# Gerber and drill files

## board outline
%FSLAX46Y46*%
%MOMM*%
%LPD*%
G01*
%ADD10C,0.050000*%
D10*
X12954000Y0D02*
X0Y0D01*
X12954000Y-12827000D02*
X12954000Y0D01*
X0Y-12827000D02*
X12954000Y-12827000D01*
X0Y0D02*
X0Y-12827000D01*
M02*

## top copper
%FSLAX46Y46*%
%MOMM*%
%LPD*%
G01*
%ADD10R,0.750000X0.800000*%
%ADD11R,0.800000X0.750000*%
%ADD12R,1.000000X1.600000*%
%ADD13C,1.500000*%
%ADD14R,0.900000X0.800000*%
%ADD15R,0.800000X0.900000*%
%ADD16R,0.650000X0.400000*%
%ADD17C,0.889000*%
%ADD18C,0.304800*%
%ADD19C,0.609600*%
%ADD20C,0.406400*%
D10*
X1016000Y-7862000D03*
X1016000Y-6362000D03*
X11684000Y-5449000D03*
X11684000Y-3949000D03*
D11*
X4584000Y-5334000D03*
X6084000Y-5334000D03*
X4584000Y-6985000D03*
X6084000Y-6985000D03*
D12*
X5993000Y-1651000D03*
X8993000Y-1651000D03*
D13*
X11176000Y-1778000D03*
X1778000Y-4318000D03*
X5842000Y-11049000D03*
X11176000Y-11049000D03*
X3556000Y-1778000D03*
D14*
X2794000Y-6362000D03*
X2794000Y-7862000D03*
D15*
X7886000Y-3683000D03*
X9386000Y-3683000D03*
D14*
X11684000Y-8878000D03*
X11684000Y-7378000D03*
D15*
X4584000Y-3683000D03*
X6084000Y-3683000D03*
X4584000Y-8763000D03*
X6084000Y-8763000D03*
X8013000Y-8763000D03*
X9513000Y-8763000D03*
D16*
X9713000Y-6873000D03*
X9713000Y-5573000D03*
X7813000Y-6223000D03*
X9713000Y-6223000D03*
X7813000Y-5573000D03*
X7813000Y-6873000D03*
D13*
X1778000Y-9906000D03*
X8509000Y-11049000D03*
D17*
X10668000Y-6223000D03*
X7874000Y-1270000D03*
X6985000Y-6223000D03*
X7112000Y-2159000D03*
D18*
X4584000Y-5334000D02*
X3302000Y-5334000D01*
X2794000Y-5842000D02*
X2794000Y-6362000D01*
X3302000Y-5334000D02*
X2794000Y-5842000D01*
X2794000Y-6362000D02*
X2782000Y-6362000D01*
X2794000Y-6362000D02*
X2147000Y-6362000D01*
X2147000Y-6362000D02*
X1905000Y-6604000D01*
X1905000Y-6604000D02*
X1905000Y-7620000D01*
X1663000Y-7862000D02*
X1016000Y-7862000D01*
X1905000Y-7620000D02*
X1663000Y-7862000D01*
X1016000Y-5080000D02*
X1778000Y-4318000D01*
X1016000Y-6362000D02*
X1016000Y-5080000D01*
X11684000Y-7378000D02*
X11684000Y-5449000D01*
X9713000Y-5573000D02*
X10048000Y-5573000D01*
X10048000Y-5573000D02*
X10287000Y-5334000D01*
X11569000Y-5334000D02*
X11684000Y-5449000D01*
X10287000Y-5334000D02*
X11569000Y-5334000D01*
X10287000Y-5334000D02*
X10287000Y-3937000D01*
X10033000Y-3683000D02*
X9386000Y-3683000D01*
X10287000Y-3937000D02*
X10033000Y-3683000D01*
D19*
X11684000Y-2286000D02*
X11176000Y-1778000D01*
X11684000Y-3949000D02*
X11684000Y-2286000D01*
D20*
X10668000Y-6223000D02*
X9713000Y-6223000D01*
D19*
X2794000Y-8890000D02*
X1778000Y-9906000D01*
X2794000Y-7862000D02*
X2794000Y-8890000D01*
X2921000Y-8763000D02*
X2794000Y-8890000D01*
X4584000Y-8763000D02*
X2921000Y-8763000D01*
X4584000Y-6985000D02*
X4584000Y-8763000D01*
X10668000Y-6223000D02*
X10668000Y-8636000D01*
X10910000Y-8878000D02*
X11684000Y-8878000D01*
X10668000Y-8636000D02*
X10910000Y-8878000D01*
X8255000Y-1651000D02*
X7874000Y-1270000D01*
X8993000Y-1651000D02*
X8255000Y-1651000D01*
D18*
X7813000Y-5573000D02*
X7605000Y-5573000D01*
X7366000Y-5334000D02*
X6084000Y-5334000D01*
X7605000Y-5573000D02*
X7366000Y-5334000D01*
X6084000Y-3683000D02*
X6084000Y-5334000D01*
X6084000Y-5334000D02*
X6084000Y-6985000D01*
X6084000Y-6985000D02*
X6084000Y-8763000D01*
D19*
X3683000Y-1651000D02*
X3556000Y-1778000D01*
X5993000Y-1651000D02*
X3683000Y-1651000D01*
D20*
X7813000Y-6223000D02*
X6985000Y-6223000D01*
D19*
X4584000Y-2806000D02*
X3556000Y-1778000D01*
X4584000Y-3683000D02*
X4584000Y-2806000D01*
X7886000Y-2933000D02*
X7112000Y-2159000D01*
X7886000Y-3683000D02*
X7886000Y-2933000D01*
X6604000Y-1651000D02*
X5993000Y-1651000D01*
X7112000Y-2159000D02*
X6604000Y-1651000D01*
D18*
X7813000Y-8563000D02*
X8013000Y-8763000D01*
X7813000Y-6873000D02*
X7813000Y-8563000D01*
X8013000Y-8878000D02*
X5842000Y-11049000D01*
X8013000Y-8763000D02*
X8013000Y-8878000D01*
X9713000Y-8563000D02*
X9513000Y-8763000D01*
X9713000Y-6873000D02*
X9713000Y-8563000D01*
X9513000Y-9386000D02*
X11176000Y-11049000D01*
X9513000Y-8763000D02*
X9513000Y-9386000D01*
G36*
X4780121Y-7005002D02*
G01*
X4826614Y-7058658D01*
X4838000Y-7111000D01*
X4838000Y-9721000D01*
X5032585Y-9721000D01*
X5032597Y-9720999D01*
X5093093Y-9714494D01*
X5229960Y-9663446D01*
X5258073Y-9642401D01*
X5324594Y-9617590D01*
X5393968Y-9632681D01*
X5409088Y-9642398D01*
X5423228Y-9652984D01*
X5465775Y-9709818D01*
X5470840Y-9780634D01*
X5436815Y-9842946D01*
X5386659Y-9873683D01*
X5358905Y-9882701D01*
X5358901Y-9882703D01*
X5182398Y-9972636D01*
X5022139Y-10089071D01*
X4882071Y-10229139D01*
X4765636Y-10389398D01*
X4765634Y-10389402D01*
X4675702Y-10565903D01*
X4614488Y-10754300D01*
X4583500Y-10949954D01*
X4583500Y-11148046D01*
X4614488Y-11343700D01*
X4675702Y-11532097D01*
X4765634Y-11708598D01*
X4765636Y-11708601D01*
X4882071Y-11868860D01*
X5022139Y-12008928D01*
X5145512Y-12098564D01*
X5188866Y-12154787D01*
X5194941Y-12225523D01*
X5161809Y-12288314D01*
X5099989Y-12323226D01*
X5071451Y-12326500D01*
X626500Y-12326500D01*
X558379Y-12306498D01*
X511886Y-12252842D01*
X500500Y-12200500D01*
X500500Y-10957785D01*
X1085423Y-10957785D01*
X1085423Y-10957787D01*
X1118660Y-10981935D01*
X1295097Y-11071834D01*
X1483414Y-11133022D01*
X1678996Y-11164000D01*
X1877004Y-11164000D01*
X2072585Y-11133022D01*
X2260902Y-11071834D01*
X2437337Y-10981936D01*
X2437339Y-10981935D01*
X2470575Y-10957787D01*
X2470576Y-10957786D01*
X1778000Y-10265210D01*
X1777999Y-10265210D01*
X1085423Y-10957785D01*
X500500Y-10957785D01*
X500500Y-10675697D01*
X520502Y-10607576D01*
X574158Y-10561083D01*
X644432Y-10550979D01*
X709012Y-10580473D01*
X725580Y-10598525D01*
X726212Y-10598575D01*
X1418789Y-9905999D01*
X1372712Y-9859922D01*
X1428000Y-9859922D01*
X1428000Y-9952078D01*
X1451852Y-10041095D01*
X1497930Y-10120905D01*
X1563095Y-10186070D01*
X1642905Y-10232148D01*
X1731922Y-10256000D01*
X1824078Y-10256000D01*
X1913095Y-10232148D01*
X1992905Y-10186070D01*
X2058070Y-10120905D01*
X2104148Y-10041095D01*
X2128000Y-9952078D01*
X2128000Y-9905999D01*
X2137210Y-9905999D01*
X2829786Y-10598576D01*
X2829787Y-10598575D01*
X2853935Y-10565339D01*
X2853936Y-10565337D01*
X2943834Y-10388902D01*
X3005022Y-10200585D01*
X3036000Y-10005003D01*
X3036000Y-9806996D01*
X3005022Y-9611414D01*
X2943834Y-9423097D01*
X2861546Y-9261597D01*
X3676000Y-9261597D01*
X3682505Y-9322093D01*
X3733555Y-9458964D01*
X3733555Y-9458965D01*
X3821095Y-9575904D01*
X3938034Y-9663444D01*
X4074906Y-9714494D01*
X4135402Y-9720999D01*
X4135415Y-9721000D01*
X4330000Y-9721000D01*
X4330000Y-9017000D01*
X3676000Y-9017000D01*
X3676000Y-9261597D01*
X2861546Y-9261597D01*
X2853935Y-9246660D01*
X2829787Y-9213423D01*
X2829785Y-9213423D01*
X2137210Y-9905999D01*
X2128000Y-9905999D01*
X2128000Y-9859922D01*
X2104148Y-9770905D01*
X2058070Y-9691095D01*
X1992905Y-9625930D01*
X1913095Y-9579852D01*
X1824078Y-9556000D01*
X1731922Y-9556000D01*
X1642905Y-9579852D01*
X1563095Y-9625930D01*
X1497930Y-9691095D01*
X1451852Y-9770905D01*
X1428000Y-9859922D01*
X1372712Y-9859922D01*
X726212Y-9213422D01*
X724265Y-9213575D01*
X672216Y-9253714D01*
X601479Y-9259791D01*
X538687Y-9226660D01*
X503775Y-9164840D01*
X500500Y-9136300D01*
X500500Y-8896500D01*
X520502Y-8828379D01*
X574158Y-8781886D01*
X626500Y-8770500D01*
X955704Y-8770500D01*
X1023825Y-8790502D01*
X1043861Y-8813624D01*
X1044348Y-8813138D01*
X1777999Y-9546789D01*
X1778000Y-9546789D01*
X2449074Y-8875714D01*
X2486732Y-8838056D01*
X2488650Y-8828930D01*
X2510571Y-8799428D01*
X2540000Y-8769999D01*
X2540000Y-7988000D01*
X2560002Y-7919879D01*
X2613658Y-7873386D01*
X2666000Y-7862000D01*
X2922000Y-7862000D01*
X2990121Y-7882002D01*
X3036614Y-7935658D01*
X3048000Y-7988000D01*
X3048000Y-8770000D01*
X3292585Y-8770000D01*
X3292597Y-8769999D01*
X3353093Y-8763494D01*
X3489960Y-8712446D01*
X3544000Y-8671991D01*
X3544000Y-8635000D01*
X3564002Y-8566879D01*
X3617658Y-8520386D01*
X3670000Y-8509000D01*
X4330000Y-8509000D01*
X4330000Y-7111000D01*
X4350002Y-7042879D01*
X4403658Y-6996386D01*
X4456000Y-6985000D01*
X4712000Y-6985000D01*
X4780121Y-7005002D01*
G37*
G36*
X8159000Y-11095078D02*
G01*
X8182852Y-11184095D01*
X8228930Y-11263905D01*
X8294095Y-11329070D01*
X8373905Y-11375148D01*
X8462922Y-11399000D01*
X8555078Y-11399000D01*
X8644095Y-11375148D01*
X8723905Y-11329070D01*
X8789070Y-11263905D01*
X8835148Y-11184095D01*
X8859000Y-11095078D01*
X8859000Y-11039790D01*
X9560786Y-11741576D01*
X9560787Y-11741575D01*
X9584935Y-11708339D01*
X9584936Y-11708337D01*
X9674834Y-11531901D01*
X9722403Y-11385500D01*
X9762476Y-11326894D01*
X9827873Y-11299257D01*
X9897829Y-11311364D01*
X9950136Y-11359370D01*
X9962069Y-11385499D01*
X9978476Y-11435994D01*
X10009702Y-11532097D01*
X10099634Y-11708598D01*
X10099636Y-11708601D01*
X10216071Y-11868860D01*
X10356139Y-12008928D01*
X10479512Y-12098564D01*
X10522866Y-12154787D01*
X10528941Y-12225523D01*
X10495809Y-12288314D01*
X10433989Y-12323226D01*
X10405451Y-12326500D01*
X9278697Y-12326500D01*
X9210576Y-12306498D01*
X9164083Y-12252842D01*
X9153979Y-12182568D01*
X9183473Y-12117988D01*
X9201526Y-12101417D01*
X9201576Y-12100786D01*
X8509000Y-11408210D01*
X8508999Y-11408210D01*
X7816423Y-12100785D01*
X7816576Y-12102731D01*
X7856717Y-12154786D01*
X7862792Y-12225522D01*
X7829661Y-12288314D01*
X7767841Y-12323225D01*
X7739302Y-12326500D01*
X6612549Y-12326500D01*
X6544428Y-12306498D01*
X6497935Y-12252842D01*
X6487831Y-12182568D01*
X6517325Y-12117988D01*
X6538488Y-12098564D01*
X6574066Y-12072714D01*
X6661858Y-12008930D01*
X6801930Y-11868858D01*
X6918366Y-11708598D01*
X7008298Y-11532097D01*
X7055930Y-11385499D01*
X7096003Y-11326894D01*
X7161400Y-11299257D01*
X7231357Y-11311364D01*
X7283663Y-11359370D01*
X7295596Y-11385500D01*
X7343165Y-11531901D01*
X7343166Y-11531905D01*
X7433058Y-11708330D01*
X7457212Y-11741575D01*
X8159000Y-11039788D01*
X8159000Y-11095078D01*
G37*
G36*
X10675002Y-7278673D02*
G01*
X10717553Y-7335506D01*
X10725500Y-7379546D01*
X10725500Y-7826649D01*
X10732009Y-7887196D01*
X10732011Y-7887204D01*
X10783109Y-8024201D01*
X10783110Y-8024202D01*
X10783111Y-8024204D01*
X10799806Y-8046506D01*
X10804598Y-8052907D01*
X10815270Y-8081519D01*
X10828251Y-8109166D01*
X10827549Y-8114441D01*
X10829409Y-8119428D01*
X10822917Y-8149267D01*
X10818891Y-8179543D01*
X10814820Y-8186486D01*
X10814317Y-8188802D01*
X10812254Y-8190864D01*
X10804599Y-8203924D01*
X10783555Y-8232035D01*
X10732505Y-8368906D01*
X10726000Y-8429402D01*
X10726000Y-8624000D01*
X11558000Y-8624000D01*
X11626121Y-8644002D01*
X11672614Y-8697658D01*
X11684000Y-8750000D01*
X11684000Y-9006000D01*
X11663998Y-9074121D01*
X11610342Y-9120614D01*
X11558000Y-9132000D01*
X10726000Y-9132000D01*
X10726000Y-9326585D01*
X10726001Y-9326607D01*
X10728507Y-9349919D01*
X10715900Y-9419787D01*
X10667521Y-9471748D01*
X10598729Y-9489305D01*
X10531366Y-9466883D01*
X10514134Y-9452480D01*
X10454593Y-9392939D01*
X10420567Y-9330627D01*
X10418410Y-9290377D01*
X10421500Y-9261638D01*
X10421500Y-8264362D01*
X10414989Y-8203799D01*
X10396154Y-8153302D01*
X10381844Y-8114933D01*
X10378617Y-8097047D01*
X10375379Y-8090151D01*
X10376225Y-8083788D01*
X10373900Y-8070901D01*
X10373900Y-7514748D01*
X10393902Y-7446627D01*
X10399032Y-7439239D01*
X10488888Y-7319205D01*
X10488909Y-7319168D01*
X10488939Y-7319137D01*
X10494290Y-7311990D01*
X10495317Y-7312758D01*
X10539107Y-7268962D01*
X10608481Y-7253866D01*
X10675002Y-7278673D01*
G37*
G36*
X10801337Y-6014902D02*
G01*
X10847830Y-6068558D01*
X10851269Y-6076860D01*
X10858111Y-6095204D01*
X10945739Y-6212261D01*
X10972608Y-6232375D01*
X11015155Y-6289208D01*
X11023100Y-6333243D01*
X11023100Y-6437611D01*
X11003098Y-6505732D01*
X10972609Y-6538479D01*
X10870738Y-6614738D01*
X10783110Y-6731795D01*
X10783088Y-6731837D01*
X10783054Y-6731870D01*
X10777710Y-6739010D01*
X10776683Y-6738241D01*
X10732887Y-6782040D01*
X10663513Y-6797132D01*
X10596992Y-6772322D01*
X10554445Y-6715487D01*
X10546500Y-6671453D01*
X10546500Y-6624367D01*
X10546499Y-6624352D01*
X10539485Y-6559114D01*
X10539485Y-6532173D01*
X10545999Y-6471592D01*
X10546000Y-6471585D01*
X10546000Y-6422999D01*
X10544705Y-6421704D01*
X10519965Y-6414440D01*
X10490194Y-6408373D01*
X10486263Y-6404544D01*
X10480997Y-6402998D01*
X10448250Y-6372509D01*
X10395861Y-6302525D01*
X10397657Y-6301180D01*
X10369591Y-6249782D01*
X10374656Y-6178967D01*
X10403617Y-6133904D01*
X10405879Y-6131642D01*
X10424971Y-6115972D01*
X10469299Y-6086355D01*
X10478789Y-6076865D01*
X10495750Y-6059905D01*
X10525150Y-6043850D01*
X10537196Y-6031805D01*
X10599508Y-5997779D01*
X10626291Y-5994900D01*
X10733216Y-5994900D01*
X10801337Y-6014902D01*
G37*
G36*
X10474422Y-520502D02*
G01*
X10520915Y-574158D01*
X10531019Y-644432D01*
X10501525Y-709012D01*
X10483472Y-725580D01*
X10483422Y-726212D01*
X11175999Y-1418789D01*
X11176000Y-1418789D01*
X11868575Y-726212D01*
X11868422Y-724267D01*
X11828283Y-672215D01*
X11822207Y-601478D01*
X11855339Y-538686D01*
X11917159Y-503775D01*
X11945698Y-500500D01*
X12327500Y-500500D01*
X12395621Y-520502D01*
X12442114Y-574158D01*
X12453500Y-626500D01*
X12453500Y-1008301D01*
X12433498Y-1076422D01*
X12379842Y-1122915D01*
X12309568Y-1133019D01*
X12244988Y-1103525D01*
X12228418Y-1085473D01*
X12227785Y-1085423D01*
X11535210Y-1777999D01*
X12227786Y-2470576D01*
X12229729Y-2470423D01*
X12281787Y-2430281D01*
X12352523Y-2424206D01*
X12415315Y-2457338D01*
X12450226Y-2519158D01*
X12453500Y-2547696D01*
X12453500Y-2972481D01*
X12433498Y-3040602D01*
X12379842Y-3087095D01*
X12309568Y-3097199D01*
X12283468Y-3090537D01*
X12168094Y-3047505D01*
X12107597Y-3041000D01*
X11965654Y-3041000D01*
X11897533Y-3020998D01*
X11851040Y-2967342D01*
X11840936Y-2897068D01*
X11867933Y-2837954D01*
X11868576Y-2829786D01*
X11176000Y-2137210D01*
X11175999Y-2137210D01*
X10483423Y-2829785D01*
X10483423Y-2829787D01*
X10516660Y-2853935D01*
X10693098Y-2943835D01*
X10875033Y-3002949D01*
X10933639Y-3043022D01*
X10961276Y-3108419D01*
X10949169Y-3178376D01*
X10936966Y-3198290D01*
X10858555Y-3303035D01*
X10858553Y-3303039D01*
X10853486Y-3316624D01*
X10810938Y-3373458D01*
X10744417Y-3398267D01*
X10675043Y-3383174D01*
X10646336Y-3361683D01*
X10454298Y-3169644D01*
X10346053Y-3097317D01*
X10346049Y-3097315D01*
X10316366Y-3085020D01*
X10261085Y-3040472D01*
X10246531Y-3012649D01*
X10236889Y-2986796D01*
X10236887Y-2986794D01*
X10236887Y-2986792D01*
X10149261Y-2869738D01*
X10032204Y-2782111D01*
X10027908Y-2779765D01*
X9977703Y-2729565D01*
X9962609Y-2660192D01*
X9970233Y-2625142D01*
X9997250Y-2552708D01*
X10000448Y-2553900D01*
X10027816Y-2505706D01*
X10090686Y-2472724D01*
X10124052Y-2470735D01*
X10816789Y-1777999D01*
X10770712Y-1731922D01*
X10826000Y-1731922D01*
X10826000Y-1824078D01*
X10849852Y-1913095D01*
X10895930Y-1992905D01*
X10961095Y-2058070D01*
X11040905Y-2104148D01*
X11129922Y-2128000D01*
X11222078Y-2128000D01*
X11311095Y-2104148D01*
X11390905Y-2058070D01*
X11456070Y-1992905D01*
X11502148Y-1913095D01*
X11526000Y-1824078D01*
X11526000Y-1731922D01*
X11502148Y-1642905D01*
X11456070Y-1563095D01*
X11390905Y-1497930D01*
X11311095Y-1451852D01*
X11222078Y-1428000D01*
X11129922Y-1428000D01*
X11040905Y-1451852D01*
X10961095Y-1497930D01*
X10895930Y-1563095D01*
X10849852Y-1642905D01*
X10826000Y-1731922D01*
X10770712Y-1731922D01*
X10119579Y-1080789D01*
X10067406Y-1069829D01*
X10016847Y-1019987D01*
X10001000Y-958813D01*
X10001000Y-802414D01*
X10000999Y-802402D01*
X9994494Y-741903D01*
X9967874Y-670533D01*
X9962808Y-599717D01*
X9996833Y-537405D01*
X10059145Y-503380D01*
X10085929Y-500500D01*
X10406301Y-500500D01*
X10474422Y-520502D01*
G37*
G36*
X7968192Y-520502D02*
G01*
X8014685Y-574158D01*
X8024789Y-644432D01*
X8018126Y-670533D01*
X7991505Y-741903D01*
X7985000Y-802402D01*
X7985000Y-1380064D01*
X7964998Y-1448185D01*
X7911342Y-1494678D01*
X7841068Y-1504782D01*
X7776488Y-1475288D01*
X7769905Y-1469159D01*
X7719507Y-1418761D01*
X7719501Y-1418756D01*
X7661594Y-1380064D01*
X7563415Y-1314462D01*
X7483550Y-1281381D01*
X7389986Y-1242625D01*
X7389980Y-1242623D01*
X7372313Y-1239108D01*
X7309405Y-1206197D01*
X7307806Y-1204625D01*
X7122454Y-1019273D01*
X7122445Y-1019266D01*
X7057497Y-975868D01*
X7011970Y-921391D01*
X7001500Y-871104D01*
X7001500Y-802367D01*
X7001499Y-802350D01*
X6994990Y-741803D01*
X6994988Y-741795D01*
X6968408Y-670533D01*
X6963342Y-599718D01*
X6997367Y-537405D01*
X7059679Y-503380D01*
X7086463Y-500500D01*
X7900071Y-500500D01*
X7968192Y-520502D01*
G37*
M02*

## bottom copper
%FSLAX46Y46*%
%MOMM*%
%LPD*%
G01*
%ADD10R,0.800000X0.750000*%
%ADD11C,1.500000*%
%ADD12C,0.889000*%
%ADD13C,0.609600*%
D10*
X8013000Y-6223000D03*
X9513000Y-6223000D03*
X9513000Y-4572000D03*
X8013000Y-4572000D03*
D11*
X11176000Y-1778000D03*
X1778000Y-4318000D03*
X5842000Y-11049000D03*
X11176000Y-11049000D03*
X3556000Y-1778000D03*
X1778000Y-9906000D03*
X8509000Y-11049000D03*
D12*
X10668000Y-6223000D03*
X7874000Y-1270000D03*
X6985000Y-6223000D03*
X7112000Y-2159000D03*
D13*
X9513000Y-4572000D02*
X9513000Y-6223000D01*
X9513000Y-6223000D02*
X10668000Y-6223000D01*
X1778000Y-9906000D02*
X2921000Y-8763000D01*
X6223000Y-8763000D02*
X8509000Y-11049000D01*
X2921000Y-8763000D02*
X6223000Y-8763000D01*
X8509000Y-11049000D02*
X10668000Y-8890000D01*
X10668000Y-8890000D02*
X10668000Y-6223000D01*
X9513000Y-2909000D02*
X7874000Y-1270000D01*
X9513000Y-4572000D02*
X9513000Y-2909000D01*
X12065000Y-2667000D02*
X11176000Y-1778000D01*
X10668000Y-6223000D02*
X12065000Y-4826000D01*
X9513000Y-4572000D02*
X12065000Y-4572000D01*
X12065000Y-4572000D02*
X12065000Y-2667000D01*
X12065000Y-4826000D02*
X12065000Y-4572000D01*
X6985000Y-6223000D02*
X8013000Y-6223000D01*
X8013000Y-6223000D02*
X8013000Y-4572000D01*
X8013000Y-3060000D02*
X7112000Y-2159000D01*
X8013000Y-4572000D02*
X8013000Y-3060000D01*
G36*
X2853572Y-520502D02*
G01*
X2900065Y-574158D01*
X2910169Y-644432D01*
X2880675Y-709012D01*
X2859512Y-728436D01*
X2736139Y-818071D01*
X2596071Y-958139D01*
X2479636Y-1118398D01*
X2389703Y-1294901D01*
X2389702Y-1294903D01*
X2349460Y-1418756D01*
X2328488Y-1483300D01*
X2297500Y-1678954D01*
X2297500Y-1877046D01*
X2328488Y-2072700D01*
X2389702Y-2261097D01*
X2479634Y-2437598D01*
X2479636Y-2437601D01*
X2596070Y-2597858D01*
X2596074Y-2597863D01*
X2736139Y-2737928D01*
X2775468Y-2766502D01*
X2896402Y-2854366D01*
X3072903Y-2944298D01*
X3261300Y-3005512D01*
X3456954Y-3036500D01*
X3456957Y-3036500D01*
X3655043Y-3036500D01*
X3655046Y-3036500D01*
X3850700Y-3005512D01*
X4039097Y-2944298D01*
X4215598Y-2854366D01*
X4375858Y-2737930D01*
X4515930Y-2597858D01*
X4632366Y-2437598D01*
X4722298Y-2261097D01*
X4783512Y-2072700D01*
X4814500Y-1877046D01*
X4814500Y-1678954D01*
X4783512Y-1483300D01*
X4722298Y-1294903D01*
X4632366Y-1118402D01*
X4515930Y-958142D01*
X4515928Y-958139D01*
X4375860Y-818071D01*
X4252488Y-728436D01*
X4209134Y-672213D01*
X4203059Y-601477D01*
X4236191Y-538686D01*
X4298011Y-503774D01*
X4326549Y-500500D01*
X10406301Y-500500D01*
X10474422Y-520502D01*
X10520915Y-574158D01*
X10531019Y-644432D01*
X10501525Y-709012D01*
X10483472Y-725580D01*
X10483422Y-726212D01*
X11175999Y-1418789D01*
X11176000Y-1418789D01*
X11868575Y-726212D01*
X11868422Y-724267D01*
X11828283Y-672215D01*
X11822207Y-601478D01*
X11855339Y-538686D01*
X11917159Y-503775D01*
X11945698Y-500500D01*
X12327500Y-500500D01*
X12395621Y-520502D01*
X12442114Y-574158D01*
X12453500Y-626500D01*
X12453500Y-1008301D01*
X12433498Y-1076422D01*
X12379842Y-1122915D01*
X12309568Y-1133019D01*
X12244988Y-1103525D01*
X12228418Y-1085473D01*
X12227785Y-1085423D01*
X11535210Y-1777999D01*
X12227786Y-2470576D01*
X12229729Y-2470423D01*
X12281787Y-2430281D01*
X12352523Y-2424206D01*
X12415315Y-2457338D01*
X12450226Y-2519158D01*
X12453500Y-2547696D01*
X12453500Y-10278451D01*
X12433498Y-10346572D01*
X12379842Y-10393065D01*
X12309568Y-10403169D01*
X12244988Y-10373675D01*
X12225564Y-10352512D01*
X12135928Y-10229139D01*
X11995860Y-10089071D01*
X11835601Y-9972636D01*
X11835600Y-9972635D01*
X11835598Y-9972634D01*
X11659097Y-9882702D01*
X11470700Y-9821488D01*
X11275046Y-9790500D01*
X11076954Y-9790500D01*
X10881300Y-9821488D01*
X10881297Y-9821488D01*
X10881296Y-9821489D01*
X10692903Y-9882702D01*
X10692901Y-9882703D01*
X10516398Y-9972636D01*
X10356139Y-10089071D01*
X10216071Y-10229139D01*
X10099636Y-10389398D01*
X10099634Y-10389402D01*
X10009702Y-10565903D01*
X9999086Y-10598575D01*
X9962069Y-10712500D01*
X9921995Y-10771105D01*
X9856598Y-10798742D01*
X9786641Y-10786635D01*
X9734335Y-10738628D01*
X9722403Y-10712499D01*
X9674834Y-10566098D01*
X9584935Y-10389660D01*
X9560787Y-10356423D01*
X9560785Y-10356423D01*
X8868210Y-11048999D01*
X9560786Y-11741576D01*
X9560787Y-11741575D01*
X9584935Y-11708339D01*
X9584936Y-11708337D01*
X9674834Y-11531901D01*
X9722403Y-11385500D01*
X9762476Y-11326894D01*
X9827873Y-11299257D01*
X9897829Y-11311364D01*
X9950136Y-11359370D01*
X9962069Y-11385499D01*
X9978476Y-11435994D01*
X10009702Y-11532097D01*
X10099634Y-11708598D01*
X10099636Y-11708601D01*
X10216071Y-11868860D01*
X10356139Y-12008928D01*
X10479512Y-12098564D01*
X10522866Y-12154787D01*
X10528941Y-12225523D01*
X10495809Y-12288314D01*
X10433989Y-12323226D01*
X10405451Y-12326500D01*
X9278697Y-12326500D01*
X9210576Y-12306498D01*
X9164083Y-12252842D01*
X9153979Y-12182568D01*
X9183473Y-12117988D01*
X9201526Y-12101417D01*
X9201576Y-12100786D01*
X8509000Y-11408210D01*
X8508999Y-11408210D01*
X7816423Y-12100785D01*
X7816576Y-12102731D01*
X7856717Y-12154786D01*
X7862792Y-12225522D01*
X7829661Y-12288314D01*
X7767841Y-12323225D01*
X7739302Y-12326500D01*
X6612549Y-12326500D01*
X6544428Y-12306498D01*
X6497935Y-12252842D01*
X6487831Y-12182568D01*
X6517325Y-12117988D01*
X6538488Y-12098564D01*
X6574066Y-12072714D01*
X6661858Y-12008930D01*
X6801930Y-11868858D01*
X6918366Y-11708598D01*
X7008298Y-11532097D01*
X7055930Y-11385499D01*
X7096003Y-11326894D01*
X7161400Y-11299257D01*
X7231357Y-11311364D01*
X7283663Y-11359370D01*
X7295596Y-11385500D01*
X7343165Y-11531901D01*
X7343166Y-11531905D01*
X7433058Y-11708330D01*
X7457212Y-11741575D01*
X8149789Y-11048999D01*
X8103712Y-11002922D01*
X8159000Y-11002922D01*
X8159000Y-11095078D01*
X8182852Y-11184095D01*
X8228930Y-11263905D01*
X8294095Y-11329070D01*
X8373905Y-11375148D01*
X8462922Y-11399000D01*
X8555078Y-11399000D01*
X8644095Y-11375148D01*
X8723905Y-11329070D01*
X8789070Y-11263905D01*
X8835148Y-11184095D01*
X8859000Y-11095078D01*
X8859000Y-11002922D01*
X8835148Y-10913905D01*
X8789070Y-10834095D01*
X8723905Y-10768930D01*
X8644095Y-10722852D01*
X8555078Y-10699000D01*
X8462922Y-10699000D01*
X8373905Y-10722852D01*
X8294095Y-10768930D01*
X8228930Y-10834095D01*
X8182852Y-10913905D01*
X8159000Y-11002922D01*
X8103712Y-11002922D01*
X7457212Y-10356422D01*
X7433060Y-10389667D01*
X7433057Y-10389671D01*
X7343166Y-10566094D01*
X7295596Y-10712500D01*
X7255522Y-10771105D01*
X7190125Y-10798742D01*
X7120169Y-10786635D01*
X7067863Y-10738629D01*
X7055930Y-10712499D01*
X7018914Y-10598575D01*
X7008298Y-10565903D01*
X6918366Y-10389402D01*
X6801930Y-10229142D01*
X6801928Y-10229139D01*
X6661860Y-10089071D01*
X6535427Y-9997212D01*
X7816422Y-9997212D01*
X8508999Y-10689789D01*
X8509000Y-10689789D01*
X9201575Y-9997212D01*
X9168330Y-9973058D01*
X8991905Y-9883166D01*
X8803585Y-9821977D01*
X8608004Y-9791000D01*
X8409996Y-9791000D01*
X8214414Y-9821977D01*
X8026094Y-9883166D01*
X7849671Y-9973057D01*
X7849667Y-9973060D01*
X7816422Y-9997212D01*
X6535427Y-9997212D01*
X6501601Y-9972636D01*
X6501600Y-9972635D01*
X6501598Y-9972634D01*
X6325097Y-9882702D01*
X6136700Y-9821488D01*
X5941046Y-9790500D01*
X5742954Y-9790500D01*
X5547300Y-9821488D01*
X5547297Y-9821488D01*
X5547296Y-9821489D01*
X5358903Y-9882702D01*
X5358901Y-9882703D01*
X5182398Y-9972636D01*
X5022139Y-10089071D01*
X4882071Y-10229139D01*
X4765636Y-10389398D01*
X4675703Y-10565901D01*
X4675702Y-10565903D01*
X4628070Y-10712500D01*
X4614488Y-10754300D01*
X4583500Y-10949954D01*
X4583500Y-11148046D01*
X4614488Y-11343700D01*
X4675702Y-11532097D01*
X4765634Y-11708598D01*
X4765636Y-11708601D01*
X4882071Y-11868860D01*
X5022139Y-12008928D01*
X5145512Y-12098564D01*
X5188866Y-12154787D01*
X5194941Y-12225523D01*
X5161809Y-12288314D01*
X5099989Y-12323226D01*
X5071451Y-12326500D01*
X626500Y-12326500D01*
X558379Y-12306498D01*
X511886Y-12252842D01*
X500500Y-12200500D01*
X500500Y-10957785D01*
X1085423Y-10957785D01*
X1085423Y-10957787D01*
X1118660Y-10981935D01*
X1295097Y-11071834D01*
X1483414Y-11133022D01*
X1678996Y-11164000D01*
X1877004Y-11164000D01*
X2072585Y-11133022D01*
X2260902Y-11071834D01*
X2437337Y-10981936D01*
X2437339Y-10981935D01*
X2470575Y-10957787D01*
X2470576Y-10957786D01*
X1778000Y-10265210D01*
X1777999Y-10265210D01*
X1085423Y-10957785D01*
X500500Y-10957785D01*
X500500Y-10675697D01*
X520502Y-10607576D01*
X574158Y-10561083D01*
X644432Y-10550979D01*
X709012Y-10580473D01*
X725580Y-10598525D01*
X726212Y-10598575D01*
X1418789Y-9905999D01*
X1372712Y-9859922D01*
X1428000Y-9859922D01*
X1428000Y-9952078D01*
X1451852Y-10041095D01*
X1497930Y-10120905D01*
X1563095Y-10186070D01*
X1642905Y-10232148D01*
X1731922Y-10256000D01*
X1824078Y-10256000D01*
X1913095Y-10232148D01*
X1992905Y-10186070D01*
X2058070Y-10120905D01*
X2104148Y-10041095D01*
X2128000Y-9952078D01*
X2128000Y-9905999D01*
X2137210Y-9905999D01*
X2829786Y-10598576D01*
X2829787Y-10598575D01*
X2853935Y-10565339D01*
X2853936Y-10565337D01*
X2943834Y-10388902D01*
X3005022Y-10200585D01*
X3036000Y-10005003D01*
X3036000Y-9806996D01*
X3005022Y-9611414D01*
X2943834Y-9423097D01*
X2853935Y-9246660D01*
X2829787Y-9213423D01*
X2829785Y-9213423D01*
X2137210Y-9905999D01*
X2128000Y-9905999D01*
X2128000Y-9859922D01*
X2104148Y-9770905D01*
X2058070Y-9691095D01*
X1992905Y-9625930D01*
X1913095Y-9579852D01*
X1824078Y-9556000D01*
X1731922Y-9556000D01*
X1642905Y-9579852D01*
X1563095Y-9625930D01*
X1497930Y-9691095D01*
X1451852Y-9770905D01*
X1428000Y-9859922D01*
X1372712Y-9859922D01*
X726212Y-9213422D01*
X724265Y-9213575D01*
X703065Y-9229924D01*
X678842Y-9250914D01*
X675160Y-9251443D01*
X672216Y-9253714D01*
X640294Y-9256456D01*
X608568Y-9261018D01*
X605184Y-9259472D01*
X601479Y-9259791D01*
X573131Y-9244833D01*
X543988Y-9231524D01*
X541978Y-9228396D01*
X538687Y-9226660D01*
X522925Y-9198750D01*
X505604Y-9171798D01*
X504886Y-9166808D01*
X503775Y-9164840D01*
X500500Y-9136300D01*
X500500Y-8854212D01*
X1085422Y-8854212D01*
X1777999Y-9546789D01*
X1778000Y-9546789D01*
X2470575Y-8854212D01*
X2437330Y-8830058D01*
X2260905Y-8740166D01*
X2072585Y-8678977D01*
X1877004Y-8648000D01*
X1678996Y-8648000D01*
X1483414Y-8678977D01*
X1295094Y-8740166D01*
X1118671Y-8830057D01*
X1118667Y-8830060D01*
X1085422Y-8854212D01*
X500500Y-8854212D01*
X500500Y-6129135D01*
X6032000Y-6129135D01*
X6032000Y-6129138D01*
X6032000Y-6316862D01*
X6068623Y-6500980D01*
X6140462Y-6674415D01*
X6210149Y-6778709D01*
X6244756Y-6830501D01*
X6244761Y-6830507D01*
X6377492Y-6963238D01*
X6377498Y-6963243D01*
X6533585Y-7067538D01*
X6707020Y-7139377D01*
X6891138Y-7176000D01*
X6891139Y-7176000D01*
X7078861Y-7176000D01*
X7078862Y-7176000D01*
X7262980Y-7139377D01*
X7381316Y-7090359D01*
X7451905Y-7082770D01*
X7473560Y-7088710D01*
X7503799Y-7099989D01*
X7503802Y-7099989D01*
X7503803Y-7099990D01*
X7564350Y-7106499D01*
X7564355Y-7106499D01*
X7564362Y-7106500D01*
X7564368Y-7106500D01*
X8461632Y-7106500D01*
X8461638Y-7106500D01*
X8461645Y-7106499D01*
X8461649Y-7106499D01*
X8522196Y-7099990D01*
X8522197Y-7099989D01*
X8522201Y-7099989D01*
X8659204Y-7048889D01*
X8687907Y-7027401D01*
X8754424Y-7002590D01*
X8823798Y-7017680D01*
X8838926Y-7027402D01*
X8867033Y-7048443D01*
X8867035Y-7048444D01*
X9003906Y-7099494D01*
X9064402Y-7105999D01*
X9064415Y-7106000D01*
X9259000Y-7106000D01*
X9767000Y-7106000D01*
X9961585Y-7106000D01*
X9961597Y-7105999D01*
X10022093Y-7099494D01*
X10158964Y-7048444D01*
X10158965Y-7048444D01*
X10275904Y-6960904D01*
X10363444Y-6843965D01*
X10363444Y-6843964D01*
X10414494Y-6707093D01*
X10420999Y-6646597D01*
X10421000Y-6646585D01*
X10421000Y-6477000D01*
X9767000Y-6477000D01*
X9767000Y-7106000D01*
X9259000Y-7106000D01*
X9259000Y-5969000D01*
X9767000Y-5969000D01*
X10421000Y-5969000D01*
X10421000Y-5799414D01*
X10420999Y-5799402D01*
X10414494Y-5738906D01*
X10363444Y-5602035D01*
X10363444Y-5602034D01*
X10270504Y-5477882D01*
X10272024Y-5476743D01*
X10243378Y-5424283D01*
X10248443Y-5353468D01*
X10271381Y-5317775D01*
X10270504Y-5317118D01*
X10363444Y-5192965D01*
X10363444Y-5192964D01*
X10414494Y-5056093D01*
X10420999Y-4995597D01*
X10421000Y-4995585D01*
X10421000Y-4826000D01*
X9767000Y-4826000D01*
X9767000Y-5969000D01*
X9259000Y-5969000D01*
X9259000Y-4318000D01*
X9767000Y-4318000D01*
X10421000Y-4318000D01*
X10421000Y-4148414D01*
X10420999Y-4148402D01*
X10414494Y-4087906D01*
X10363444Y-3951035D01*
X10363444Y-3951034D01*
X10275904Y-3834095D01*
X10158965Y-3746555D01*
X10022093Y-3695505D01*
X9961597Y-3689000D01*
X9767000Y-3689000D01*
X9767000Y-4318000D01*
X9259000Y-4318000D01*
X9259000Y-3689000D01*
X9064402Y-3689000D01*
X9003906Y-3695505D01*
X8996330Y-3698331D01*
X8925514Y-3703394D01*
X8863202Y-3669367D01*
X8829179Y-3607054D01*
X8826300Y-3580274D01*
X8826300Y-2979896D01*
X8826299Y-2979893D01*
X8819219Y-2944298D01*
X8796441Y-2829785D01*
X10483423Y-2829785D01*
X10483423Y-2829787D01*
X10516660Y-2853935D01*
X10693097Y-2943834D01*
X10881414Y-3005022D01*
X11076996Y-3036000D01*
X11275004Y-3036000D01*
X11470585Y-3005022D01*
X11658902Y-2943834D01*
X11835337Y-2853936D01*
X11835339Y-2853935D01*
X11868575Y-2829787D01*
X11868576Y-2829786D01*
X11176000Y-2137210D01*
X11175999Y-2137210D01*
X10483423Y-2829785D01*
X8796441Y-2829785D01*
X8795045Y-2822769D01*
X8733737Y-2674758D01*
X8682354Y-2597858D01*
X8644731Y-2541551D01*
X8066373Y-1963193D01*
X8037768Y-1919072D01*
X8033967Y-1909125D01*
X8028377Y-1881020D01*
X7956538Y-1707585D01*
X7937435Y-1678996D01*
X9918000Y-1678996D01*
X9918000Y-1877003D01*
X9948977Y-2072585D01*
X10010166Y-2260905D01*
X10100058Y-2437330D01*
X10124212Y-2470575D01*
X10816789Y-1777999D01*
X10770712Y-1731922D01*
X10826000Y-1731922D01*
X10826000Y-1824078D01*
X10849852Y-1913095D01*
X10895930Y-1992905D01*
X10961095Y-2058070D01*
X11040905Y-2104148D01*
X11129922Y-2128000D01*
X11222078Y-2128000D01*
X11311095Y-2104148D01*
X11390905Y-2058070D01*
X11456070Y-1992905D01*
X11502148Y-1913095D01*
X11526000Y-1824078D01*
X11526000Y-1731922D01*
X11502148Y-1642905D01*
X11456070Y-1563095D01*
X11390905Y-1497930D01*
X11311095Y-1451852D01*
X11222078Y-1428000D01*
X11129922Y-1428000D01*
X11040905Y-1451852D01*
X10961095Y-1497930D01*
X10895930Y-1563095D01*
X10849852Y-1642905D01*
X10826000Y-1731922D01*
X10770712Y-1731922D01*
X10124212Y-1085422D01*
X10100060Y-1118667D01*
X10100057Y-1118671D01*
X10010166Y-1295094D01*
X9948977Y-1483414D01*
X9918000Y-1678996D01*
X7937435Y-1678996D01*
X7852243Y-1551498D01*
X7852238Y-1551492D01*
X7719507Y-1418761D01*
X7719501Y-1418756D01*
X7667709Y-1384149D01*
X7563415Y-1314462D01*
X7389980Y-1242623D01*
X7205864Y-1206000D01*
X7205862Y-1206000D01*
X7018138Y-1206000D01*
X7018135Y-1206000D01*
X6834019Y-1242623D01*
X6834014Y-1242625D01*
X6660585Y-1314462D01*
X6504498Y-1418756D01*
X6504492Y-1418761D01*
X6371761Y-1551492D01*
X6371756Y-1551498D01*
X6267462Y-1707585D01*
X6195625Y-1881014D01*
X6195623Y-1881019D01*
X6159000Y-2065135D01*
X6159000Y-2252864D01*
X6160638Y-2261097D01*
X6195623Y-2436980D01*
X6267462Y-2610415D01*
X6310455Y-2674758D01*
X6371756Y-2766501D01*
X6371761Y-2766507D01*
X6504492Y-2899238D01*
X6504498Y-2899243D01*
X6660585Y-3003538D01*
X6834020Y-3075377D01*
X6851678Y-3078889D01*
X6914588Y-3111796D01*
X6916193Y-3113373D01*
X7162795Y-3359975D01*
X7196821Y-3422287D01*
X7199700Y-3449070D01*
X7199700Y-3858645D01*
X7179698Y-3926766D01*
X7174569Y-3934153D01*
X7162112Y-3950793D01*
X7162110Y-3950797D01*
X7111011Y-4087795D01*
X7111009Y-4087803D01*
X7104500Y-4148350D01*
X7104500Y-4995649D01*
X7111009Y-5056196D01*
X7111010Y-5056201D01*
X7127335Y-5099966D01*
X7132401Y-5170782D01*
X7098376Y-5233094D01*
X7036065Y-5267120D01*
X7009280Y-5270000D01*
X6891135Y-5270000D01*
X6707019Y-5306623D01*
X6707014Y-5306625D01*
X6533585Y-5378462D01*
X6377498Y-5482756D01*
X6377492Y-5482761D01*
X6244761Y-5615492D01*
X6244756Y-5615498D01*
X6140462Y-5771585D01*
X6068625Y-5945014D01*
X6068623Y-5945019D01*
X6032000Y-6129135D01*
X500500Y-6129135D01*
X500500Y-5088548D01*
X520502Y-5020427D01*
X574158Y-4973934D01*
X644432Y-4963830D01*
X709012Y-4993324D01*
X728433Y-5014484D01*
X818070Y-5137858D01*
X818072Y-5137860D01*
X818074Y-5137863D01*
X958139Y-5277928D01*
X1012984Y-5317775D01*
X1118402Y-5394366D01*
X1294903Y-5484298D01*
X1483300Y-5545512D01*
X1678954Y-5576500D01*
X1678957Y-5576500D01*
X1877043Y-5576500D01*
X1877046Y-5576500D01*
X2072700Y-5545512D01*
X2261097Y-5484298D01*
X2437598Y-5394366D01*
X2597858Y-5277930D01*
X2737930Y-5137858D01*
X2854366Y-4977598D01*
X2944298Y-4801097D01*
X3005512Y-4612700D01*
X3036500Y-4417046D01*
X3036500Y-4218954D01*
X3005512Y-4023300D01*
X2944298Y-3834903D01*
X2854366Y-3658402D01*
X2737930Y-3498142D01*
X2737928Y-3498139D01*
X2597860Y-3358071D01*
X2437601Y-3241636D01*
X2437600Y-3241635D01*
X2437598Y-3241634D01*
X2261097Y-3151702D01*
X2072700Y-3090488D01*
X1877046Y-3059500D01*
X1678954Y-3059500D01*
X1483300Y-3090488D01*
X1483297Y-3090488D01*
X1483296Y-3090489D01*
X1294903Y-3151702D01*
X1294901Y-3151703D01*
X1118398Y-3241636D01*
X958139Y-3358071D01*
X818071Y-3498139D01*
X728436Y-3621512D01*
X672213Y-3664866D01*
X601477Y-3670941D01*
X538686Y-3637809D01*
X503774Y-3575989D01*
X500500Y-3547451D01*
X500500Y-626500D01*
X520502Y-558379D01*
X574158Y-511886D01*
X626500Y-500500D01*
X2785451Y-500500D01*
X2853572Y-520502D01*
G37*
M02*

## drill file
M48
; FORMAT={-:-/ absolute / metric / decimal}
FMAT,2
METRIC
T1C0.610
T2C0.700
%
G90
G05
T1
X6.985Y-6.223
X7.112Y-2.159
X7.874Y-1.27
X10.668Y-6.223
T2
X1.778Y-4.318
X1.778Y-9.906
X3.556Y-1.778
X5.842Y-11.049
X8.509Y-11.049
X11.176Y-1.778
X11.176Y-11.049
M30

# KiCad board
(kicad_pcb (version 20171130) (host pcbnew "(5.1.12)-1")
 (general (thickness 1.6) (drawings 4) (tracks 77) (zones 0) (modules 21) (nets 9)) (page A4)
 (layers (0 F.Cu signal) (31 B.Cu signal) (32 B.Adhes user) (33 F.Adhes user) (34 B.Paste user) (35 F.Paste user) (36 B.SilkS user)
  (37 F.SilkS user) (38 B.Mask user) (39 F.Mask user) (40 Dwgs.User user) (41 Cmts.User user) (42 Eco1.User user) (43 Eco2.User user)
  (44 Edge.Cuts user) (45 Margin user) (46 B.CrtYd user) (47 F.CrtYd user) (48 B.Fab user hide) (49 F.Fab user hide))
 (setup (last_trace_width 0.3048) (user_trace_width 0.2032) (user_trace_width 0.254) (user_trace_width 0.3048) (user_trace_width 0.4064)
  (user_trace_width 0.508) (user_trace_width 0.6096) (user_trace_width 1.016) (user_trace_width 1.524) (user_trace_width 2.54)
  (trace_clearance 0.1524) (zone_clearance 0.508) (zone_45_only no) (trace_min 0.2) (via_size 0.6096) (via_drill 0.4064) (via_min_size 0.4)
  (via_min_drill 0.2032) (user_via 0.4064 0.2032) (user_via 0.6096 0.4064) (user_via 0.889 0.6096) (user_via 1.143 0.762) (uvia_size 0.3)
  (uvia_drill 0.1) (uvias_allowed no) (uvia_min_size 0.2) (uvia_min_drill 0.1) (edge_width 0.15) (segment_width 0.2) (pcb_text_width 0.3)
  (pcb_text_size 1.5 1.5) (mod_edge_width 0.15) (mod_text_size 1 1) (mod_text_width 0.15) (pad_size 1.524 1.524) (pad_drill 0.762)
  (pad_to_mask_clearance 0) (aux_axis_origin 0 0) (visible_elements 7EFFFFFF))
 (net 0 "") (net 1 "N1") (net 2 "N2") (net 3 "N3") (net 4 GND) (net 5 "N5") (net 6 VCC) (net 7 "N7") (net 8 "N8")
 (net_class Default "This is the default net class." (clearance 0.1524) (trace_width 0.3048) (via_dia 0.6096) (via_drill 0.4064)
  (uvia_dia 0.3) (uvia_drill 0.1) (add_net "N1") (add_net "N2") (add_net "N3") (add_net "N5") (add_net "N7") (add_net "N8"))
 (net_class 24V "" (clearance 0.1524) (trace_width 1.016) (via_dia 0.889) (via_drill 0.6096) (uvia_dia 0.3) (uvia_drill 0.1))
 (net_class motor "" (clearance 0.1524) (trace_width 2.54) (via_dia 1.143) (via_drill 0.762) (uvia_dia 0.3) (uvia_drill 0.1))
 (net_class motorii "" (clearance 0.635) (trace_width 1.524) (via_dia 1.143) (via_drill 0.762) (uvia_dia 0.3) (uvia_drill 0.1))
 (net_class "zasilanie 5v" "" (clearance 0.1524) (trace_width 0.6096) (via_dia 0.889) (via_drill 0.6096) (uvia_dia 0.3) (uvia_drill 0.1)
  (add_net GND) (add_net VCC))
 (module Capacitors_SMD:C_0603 (layer F.Cu) (at 1.016 7.112 90)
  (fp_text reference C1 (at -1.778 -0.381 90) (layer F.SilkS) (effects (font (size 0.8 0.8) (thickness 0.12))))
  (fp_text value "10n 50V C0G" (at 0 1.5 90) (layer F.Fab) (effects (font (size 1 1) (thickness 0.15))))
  (pad 1 smd rect (at -0.75 0 90) (size 0.8 0.75) (layers F.Cu F.Paste F.Mask) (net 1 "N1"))
  (pad 2 smd rect (at 0.75 0 90) (size 0.8 0.75) (layers F.Cu F.Paste F.Mask) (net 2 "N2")))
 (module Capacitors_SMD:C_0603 (layer F.Cu) (at 11.684 4.699 90)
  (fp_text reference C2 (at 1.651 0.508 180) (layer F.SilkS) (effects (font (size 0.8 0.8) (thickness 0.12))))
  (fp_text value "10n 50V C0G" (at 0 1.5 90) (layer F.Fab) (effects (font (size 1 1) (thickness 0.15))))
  (pad 1 smd rect (at -0.75 0 90) (size 0.8 0.75) (layers F.Cu F.Paste F.Mask) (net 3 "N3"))
  (pad 2 smd rect (at 0.75 0 90) (size 0.8 0.75) (layers F.Cu F.Paste F.Mask) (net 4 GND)))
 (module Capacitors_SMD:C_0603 (layer F.Cu) (at 5.334 5.334 180)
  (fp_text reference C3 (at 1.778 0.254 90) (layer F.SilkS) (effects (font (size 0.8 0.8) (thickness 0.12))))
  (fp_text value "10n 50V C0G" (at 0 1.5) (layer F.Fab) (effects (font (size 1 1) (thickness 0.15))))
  (pad 2 smd rect (at 0.75 0 180) (size 0.8 0.75) (layers F.Cu F.Paste F.Mask) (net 1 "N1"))
  (pad 1 smd rect (at -0.75 0 180) (size 0.8 0.75) (layers F.Cu F.Paste F.Mask) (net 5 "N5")))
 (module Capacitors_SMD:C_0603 (layer F.Cu) (at 5.334 6.985 180)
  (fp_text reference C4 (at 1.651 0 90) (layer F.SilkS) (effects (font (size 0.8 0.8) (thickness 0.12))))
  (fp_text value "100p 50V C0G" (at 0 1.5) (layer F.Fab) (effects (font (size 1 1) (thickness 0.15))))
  (pad 2 smd rect (at 0.75 0 180) (size 0.8 0.75) (layers F.Cu F.Paste F.Mask) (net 4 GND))
  (pad 1 smd rect (at -0.75 0 180) (size 0.8 0.75) (layers F.Cu F.Paste F.Mask) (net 5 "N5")))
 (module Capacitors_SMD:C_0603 (layer B.Cu) (at 8.763 6.223)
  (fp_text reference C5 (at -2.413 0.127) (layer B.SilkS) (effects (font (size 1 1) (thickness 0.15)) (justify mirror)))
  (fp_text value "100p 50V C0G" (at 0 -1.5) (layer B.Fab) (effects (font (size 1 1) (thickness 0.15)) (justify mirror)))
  (pad 1 smd rect (at -0.75 0) (size 0.8 0.75) (layers B.Cu B.Paste B.Mask) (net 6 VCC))
  (pad 2 smd rect (at 0.75 0) (size 0.8 0.75) (layers B.Cu B.Paste B.Mask) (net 4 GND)))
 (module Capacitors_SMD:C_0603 (layer B.Cu) (at 8.763 4.572)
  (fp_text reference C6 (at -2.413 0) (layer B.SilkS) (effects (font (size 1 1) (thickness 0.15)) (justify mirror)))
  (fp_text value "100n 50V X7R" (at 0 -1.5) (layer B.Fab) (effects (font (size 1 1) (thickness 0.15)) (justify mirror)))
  (pad 2 smd rect (at 0.75 0) (size 0.8 0.75) (layers B.Cu B.Paste B.Mask) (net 4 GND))
  (pad 1 smd rect (at -0.75 0) (size 0.8 0.75) (layers B.Cu B.Paste B.Mask) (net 6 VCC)))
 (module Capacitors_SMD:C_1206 (layer F.Cu) (at 7.493 1.651)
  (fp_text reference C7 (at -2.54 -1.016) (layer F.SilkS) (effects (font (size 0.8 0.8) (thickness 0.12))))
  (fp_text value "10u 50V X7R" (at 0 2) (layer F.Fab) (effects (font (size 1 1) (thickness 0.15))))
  (pad 1 smd rect (at -1.5 0) (size 1 1.6) (layers F.Cu F.Paste F.Mask) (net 6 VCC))
  (pad 2 smd rect (at 1.5 0) (size 1 1.6) (layers F.Cu F.Paste F.Mask) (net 4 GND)))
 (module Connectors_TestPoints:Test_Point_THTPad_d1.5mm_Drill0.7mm (layer F.Cu) (at 11.176 1.778)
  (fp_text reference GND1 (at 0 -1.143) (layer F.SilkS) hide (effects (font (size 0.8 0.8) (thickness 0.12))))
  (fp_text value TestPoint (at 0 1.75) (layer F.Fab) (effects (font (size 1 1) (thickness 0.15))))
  (pad 1 thru_hole circle (at 0 0) (size 1.5 1.5) (drill 0.7) (layers *.Cu *.Mask) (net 4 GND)))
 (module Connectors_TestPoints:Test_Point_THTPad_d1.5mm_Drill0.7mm (layer F.Cu) (at 1.778 4.318)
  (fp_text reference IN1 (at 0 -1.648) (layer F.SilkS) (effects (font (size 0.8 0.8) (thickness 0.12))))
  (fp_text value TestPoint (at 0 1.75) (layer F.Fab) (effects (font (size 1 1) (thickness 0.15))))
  (pad 1 thru_hole circle (at 0 0) (size 1.5 1.5) (drill 0.7) (layers *.Cu *.Mask) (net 2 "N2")))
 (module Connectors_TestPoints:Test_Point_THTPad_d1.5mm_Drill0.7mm (layer F.Cu) (at 5.842 11.049)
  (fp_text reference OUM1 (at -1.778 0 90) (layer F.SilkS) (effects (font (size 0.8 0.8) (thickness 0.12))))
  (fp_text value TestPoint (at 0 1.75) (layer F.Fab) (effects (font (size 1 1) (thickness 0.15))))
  (pad 1 thru_hole circle (at 0 0) (size 1.5 1.5) (drill 0.7) (layers *.Cu *.Mask) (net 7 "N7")))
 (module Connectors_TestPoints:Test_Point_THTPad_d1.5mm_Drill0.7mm (layer F.Cu) (at 11.176 11.049)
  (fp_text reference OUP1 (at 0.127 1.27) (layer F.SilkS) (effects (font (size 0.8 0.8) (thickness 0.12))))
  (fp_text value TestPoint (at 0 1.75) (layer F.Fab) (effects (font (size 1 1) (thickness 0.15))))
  (pad 1 thru_hole circle (at 0 0) (size 1.5 1.5) (drill 0.7) (layers *.Cu *.Mask) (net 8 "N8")))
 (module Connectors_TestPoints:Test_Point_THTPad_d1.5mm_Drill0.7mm (layer F.Cu) (at 3.556 1.778)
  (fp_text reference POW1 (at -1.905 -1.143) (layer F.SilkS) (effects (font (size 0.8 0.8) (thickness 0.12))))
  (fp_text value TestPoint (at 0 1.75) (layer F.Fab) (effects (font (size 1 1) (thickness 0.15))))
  (pad 1 thru_hole circle (at 0 0) (size 1.5 1.5) (drill 0.7) (layers *.Cu *.Mask) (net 6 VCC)))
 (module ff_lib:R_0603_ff (layer F.Cu) (at 2.794 7.112 270)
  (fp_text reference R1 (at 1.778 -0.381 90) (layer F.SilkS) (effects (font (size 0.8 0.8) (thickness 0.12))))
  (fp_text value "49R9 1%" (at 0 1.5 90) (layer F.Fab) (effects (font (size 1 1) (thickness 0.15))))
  (pad 1 smd rect (at -0.75 0 270) (size 0.8 0.9) (layers F.Cu F.Paste F.Mask) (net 1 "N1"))
  (pad 2 smd rect (at 0.75 0 270) (size 0.8 0.9) (layers F.Cu F.Paste F.Mask) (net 4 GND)))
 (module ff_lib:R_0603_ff (layer F.Cu) (at 8.636 3.683)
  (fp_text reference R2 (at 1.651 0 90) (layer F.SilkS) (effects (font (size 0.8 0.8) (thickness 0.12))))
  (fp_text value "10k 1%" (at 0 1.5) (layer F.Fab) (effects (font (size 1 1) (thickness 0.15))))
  (pad 1 smd rect (at -0.75 0) (size 0.8 0.9) (layers F.Cu F.Paste F.Mask) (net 6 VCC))
  (pad 2 smd rect (at 0.75 0) (size 0.8 0.9) (layers F.Cu F.Paste F.Mask) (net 3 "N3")))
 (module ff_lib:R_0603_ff (layer F.Cu) (at 11.684 8.128 270)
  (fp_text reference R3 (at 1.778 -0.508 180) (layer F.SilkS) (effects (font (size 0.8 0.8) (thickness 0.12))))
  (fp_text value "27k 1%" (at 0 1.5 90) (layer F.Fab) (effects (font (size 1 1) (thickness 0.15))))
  (pad 2 smd rect (at 0.75 0 270) (size 0.8 0.9) (layers F.Cu F.Paste F.Mask) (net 4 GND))
  (pad 1 smd rect (at -0.75 0 270) (size 0.8 0.9) (layers F.Cu F.Paste F.Mask) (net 3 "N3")))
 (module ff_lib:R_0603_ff (layer F.Cu) (at 5.334 3.683)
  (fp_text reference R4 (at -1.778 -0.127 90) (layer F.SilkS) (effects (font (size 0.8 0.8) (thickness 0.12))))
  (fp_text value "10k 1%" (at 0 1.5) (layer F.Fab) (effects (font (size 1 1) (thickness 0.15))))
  (pad 1 smd rect (at -0.75 0) (size 0.8 0.9) (layers F.Cu F.Paste F.Mask) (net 6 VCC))
  (pad 2 smd rect (at 0.75 0) (size 0.8 0.9) (layers F.Cu F.Paste F.Mask) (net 5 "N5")))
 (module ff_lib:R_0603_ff (layer F.Cu) (at 5.334 8.763 180)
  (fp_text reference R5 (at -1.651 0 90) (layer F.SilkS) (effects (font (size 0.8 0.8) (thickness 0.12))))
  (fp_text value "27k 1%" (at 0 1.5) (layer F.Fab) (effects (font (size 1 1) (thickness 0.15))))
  (pad 2 smd rect (at 0.75 0 180) (size 0.8 0.9) (layers F.Cu F.Paste F.Mask) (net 4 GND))
  (pad 1 smd rect (at -0.75 0 180) (size 0.8 0.9) (layers F.Cu F.Paste F.Mask) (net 5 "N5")))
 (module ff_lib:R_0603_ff (layer F.Cu) (at 8.763 8.763 180)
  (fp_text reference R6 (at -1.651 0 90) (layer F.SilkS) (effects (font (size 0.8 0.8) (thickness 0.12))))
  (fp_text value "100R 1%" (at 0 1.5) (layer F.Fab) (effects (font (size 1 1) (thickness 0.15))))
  (pad 2 smd rect (at 0.75 0 180) (size 0.8 0.9) (layers F.Cu F.Paste F.Mask) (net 7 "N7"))
  (pad 1 smd rect (at -0.75 0 180) (size 0.8 0.9) (layers F.Cu F.Paste F.Mask) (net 8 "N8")))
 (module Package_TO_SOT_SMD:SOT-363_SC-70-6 (layer F.Cu) (at 8.763 6.223 180)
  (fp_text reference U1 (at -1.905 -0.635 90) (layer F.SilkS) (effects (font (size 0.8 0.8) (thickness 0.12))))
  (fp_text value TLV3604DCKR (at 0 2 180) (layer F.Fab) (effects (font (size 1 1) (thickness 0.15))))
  (pad 1 smd rect (at -0.95 -0.65 180) (size 0.65 0.4) (layers F.Cu F.Paste F.Mask) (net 8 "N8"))
  (pad 3 smd rect (at -0.95 0.65 180) (size 0.65 0.4) (layers F.Cu F.Paste F.Mask) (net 3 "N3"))
  (pad 5 smd rect (at 0.95 0 180) (size 0.65 0.4) (layers F.Cu F.Paste F.Mask) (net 6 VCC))
  (pad 2 smd rect (at -0.95 0 180) (size 0.65 0.4) (layers F.Cu F.Paste F.Mask) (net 4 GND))
  (pad 4 smd rect (at 0.95 0.65 180) (size 0.65 0.4) (layers F.Cu F.Paste F.Mask) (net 5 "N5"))
  (pad 6 smd rect (at 0.95 -0.65 180) (size 0.65 0.4) (layers F.Cu F.Paste F.Mask) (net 7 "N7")))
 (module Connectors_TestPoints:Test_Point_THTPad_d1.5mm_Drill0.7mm (layer F.Cu) (at 1.778 9.906)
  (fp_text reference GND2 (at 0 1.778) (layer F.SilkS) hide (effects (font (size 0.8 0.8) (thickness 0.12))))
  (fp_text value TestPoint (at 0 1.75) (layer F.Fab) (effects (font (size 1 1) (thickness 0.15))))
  (pad 1 thru_hole circle (at 0 0) (size 1.5 1.5) (drill 0.7) (layers *.Cu *.Mask) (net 4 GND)))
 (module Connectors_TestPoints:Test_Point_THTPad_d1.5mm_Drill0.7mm (layer F.Cu) (at 8.509 11.049)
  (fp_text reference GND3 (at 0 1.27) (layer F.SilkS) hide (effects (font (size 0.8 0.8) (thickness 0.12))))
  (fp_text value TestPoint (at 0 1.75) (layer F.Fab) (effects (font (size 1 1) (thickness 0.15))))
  (pad 1 thru_hole circle (at 0 0) (size 1.5 1.5) (drill 0.7) (layers *.Cu *.Mask) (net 4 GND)))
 (gr_line (start 12.954 0) (end 0 0) (layer Edge.Cuts) (width 0.05))
 (gr_line (start 12.954 12.827) (end 12.954 0) (layer Edge.Cuts) (width 0.05))
 (gr_line (start 0 12.827) (end 12.954 12.827) (layer Edge.Cuts) (width 0.05))
 (gr_line (start 0 0) (end 0 12.827) (layer Edge.Cuts) (width 0.05))
 (segment (start 4.584 5.334) (end 3.302 5.334) (width 0.3048) (layer F.Cu) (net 1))
 (segment (start 2.794 5.842) (end 2.794 6.362) (width 0.3048) (layer F.Cu) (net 1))
 (segment (start 3.302 5.334) (end 2.794 5.842) (width 0.3048) (layer F.Cu) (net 1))
 (segment (start 2.794 6.362) (end 2.782 6.362) (width 0.3048) (layer F.Cu) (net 1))
 (segment (start 2.794 6.362) (end 2.147 6.362) (width 0.3048) (layer F.Cu) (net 1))
 (segment (start 2.147 6.362) (end 1.905 6.604) (width 0.3048) (layer F.Cu) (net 1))
 (segment (start 1.905 6.604) (end 1.905 7.62) (width 0.3048) (layer F.Cu) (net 1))
 (segment (start 1.663 7.862) (end 1.016 7.862) (width 0.3048) (layer F.Cu) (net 1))
 (segment (start 1.905 7.62) (end 1.663 7.862) (width 0.3048) (layer F.Cu) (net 1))
 (segment (start 1.016 5.08) (end 1.778 4.318) (width 0.3048) (layer F.Cu) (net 2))
 (segment (start 1.016 6.362) (end 1.016 5.08) (width 0.3048) (layer F.Cu) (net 2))
 (segment (start 11.684 7.378) (end 11.684 5.449) (width 0.3048) (layer F.Cu) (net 3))
 (segment (start 9.713 5.573) (end 10.048 5.573) (width 0.3048) (layer F.Cu) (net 3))
 (segment (start 10.048 5.573) (end 10.287 5.334) (width 0.3048) (layer F.Cu) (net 3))
 (segment (start 11.569 5.334) (end 11.684 5.449) (width 0.3048) (layer F.Cu) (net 3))
 (segment (start 10.287 5.334) (end 11.569 5.334) (width 0.3048) (layer F.Cu) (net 3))
 (segment (start 10.287 5.334) (end 10.287 3.937) (width 0.3048) (layer F.Cu) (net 3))
 (segment (start 10.033 3.683) (end 9.386 3.683) (width 0.3048) (layer F.Cu) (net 3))
 (segment (start 10.287 3.937) (end 10.033 3.683) (width 0.3048) (layer F.Cu) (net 3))
 (segment (start 11.684 2.286) (end 11.176 1.778) (width 0.6096) (layer F.Cu) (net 4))
 (segment (start 11.684 3.949) (end 11.684 2.286) (width 0.6096) (layer F.Cu) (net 4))
 (segment (start 9.513 4.572) (end 9.513 6.223) (width 0.6096) (layer B.Cu) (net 4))
 (via (at 10.668 6.223) (size 0.889) (drill 0.6096) (layers F.Cu B.Cu) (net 4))
 (segment (start 9.513 6.223) (end 10.668 6.223) (width 0.6096) (layer B.Cu) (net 4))
 (segment (start 10.668 6.223) (end 9.713 6.223) (width 0.4064) (layer F.Cu) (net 4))
 (segment (start 2.794 8.89) (end 1.778 9.906) (width 0.6096) (layer F.Cu) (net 4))
 (segment (start 2.794 7.862) (end 2.794 8.89) (width 0.6096) (layer F.Cu) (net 4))
 (segment (start 2.921 8.763) (end 2.794 8.89) (width 0.6096) (layer F.Cu) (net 4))
 (segment (start 4.584 8.763) (end 2.921 8.763) (width 0.6096) (layer F.Cu) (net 4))
 (segment (start 4.584 6.985) (end 4.584 8.763) (width 0.6096) (layer F.Cu) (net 4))
 (segment (start 1.778 9.906) (end 2.921 8.763) (width 0.6096) (layer B.Cu) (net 4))
 (segment (start 6.223 8.763) (end 8.509 11.049) (width 0.6096) (layer B.Cu) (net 4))
 (segment (start 2.921 8.763) (end 6.223 8.763) (width 0.6096) (layer B.Cu) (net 4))
 (segment (start 8.509 11.049) (end 10.668 8.89) (width 0.6096) (layer B.Cu) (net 4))
 (segment (start 10.668 8.89) (end 10.668 6.223) (width 0.6096) (layer B.Cu) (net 4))
 (segment (start 10.668 6.223) (end 10.668 8.636) (width 0.6096) (layer F.Cu) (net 4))
 (segment (start 10.91 8.878) (end 11.684 8.878) (width 0.6096) (layer F.Cu) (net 4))
 (segment (start 10.668 8.636) (end 10.91 8.878) (width 0.6096) (layer F.Cu) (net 4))
 (segment (start 9.513 2.909) (end 7.874 1.27) (width 0.6096) (layer B.Cu) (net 4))
 (segment (start 8.255 1.651) (end 7.874 1.27) (width 0.6096) (layer F.Cu) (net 4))
 (segment (start 8.993 1.651) (end 8.255 1.651) (width 0.6096) (layer F.Cu) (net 4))
 (segment (start 9.513 4.572) (end 9.513 2.909) (width 0.6096) (layer B.Cu) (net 4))
 (via (at 7.874 1.27) (size 0.889) (drill 0.6096) (layers F.Cu B.Cu) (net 4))
 (segment (start 12.065 2.667) (end 11.176 1.778) (width 0.6096) (layer B.Cu) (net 4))
 (segment (start 10.668 6.223) (end 12.065 4.826) (width 0.6096) (layer B.Cu) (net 4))
 (segment (start 9.513 4.572) (end 12.065 4.572) (width 0.6096) (layer B.Cu) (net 4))
 (segment (start 12.065 4.572) (end 12.065 2.667) (width 0.6096) (layer B.Cu) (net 4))
 (segment (start 12.065 4.826) (end 12.065 4.572) (width 0.6096) (layer B.Cu) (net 4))
 (segment (start 7.813 5.573) (end 7.605 5.573) (width 0.3048) (layer F.Cu) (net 5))
 (segment (start 7.366 5.334) (end 6.084 5.334) (width 0.3048) (layer F.Cu) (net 5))
 (segment (start 7.605 5.573) (end 7.366 5.334) (width 0.3048) (layer F.Cu) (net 5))
 (segment (start 6.084 3.683) (end 6.084 5.334) (width 0.3048) (layer F.Cu) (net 5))
 (segment (start 6.084 5.334) (end 6.084 6.985) (width 0.3048) (layer F.Cu) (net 5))
 (segment (start 6.084 6.985) (end 6.084 8.763) (width 0.3048) (layer F.Cu) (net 5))
 (segment (start 3.683 1.651) (end 3.556 1.778) (width 0.6096) (layer F.Cu) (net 6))
 (segment (start 5.993 1.651) (end 3.683 1.651) (width 0.6096) (layer F.Cu) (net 6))
 (via (at 6.985 6.223) (size 0.889) (drill 0.6096) (layers F.Cu B.Cu) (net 6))
 (segment (start 7.813 6.223) (end 6.985 6.223) (width 0.4064) (layer F.Cu) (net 6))
 (segment (start 6.985 6.223) (end 8.013 6.223) (width 0.6096) (layer B.Cu) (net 6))
 (segment (start 8.013 6.223) (end 8.013 4.572) (width 0.6096) (layer B.Cu) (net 6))
 (via (at 7.112 2.159) (size 0.889) (drill 0.6096) (layers F.Cu B.Cu) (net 6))
 (segment (start 4.584 2.806) (end 3.556 1.778) (width 0.6096) (layer F.Cu) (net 6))
 (segment (start 4.584 3.683) (end 4.584 2.806) (width 0.6096) (layer F.Cu) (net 6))
 (segment (start 7.886 2.933) (end 7.112 2.159) (width 0.6096) (layer F.Cu) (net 6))
 (segment (start 7.886 3.683) (end 7.886 2.933) (width 0.6096) (layer F.Cu) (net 6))
 (segment (start 6.604 1.651) (end 5.993 1.651) (width 0.6096) (layer F.Cu) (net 6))
 (segment (start 7.112 2.159) (end 6.604 1.651) (width 0.6096) (layer F.Cu) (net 6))
 (segment (start 8.013 3.06) (end 7.112 2.159) (width 0.6096) (layer B.Cu) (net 6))
 (segment (start 8.013 4.572) (end 8.013 3.06) (width 0.6096) (layer B.Cu) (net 6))
 (segment (start 7.813 8.563) (end 8.013 8.763) (width 0.3048) (layer F.Cu) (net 7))
 (segment (start 7.813 6.873) (end 7.813 8.563) (width 0.3048) (layer F.Cu) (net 7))
 (segment (start 8.013 8.878) (end 5.842 11.049) (width 0.3048) (layer F.Cu) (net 7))
 (segment (start 8.013 8.763) (end 8.013 8.878) (width 0.3048) (layer F.Cu) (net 7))
 (segment (start 9.713 8.563) (end 9.513 8.763) (width 0.3048) (layer F.Cu) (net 8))
 (segment (start 9.713 6.873) (end 9.713 8.563) (width 0.3048) (layer F.Cu) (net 8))
 (segment (start 9.513 9.386) (end 11.176 11.049) (width 0.3048) (layer F.Cu) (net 8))
 (segment (start 9.513 8.763) (end 9.513 9.386) (width 0.3048) (layer F.Cu) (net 8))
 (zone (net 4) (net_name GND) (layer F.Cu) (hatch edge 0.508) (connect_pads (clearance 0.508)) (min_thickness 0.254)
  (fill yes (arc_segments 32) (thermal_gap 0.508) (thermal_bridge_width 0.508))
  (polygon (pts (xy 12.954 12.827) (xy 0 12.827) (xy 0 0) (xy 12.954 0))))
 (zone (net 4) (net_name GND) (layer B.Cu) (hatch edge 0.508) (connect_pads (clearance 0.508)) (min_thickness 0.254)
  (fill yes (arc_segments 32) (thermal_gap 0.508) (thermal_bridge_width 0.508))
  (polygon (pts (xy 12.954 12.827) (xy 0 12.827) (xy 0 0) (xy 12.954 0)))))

